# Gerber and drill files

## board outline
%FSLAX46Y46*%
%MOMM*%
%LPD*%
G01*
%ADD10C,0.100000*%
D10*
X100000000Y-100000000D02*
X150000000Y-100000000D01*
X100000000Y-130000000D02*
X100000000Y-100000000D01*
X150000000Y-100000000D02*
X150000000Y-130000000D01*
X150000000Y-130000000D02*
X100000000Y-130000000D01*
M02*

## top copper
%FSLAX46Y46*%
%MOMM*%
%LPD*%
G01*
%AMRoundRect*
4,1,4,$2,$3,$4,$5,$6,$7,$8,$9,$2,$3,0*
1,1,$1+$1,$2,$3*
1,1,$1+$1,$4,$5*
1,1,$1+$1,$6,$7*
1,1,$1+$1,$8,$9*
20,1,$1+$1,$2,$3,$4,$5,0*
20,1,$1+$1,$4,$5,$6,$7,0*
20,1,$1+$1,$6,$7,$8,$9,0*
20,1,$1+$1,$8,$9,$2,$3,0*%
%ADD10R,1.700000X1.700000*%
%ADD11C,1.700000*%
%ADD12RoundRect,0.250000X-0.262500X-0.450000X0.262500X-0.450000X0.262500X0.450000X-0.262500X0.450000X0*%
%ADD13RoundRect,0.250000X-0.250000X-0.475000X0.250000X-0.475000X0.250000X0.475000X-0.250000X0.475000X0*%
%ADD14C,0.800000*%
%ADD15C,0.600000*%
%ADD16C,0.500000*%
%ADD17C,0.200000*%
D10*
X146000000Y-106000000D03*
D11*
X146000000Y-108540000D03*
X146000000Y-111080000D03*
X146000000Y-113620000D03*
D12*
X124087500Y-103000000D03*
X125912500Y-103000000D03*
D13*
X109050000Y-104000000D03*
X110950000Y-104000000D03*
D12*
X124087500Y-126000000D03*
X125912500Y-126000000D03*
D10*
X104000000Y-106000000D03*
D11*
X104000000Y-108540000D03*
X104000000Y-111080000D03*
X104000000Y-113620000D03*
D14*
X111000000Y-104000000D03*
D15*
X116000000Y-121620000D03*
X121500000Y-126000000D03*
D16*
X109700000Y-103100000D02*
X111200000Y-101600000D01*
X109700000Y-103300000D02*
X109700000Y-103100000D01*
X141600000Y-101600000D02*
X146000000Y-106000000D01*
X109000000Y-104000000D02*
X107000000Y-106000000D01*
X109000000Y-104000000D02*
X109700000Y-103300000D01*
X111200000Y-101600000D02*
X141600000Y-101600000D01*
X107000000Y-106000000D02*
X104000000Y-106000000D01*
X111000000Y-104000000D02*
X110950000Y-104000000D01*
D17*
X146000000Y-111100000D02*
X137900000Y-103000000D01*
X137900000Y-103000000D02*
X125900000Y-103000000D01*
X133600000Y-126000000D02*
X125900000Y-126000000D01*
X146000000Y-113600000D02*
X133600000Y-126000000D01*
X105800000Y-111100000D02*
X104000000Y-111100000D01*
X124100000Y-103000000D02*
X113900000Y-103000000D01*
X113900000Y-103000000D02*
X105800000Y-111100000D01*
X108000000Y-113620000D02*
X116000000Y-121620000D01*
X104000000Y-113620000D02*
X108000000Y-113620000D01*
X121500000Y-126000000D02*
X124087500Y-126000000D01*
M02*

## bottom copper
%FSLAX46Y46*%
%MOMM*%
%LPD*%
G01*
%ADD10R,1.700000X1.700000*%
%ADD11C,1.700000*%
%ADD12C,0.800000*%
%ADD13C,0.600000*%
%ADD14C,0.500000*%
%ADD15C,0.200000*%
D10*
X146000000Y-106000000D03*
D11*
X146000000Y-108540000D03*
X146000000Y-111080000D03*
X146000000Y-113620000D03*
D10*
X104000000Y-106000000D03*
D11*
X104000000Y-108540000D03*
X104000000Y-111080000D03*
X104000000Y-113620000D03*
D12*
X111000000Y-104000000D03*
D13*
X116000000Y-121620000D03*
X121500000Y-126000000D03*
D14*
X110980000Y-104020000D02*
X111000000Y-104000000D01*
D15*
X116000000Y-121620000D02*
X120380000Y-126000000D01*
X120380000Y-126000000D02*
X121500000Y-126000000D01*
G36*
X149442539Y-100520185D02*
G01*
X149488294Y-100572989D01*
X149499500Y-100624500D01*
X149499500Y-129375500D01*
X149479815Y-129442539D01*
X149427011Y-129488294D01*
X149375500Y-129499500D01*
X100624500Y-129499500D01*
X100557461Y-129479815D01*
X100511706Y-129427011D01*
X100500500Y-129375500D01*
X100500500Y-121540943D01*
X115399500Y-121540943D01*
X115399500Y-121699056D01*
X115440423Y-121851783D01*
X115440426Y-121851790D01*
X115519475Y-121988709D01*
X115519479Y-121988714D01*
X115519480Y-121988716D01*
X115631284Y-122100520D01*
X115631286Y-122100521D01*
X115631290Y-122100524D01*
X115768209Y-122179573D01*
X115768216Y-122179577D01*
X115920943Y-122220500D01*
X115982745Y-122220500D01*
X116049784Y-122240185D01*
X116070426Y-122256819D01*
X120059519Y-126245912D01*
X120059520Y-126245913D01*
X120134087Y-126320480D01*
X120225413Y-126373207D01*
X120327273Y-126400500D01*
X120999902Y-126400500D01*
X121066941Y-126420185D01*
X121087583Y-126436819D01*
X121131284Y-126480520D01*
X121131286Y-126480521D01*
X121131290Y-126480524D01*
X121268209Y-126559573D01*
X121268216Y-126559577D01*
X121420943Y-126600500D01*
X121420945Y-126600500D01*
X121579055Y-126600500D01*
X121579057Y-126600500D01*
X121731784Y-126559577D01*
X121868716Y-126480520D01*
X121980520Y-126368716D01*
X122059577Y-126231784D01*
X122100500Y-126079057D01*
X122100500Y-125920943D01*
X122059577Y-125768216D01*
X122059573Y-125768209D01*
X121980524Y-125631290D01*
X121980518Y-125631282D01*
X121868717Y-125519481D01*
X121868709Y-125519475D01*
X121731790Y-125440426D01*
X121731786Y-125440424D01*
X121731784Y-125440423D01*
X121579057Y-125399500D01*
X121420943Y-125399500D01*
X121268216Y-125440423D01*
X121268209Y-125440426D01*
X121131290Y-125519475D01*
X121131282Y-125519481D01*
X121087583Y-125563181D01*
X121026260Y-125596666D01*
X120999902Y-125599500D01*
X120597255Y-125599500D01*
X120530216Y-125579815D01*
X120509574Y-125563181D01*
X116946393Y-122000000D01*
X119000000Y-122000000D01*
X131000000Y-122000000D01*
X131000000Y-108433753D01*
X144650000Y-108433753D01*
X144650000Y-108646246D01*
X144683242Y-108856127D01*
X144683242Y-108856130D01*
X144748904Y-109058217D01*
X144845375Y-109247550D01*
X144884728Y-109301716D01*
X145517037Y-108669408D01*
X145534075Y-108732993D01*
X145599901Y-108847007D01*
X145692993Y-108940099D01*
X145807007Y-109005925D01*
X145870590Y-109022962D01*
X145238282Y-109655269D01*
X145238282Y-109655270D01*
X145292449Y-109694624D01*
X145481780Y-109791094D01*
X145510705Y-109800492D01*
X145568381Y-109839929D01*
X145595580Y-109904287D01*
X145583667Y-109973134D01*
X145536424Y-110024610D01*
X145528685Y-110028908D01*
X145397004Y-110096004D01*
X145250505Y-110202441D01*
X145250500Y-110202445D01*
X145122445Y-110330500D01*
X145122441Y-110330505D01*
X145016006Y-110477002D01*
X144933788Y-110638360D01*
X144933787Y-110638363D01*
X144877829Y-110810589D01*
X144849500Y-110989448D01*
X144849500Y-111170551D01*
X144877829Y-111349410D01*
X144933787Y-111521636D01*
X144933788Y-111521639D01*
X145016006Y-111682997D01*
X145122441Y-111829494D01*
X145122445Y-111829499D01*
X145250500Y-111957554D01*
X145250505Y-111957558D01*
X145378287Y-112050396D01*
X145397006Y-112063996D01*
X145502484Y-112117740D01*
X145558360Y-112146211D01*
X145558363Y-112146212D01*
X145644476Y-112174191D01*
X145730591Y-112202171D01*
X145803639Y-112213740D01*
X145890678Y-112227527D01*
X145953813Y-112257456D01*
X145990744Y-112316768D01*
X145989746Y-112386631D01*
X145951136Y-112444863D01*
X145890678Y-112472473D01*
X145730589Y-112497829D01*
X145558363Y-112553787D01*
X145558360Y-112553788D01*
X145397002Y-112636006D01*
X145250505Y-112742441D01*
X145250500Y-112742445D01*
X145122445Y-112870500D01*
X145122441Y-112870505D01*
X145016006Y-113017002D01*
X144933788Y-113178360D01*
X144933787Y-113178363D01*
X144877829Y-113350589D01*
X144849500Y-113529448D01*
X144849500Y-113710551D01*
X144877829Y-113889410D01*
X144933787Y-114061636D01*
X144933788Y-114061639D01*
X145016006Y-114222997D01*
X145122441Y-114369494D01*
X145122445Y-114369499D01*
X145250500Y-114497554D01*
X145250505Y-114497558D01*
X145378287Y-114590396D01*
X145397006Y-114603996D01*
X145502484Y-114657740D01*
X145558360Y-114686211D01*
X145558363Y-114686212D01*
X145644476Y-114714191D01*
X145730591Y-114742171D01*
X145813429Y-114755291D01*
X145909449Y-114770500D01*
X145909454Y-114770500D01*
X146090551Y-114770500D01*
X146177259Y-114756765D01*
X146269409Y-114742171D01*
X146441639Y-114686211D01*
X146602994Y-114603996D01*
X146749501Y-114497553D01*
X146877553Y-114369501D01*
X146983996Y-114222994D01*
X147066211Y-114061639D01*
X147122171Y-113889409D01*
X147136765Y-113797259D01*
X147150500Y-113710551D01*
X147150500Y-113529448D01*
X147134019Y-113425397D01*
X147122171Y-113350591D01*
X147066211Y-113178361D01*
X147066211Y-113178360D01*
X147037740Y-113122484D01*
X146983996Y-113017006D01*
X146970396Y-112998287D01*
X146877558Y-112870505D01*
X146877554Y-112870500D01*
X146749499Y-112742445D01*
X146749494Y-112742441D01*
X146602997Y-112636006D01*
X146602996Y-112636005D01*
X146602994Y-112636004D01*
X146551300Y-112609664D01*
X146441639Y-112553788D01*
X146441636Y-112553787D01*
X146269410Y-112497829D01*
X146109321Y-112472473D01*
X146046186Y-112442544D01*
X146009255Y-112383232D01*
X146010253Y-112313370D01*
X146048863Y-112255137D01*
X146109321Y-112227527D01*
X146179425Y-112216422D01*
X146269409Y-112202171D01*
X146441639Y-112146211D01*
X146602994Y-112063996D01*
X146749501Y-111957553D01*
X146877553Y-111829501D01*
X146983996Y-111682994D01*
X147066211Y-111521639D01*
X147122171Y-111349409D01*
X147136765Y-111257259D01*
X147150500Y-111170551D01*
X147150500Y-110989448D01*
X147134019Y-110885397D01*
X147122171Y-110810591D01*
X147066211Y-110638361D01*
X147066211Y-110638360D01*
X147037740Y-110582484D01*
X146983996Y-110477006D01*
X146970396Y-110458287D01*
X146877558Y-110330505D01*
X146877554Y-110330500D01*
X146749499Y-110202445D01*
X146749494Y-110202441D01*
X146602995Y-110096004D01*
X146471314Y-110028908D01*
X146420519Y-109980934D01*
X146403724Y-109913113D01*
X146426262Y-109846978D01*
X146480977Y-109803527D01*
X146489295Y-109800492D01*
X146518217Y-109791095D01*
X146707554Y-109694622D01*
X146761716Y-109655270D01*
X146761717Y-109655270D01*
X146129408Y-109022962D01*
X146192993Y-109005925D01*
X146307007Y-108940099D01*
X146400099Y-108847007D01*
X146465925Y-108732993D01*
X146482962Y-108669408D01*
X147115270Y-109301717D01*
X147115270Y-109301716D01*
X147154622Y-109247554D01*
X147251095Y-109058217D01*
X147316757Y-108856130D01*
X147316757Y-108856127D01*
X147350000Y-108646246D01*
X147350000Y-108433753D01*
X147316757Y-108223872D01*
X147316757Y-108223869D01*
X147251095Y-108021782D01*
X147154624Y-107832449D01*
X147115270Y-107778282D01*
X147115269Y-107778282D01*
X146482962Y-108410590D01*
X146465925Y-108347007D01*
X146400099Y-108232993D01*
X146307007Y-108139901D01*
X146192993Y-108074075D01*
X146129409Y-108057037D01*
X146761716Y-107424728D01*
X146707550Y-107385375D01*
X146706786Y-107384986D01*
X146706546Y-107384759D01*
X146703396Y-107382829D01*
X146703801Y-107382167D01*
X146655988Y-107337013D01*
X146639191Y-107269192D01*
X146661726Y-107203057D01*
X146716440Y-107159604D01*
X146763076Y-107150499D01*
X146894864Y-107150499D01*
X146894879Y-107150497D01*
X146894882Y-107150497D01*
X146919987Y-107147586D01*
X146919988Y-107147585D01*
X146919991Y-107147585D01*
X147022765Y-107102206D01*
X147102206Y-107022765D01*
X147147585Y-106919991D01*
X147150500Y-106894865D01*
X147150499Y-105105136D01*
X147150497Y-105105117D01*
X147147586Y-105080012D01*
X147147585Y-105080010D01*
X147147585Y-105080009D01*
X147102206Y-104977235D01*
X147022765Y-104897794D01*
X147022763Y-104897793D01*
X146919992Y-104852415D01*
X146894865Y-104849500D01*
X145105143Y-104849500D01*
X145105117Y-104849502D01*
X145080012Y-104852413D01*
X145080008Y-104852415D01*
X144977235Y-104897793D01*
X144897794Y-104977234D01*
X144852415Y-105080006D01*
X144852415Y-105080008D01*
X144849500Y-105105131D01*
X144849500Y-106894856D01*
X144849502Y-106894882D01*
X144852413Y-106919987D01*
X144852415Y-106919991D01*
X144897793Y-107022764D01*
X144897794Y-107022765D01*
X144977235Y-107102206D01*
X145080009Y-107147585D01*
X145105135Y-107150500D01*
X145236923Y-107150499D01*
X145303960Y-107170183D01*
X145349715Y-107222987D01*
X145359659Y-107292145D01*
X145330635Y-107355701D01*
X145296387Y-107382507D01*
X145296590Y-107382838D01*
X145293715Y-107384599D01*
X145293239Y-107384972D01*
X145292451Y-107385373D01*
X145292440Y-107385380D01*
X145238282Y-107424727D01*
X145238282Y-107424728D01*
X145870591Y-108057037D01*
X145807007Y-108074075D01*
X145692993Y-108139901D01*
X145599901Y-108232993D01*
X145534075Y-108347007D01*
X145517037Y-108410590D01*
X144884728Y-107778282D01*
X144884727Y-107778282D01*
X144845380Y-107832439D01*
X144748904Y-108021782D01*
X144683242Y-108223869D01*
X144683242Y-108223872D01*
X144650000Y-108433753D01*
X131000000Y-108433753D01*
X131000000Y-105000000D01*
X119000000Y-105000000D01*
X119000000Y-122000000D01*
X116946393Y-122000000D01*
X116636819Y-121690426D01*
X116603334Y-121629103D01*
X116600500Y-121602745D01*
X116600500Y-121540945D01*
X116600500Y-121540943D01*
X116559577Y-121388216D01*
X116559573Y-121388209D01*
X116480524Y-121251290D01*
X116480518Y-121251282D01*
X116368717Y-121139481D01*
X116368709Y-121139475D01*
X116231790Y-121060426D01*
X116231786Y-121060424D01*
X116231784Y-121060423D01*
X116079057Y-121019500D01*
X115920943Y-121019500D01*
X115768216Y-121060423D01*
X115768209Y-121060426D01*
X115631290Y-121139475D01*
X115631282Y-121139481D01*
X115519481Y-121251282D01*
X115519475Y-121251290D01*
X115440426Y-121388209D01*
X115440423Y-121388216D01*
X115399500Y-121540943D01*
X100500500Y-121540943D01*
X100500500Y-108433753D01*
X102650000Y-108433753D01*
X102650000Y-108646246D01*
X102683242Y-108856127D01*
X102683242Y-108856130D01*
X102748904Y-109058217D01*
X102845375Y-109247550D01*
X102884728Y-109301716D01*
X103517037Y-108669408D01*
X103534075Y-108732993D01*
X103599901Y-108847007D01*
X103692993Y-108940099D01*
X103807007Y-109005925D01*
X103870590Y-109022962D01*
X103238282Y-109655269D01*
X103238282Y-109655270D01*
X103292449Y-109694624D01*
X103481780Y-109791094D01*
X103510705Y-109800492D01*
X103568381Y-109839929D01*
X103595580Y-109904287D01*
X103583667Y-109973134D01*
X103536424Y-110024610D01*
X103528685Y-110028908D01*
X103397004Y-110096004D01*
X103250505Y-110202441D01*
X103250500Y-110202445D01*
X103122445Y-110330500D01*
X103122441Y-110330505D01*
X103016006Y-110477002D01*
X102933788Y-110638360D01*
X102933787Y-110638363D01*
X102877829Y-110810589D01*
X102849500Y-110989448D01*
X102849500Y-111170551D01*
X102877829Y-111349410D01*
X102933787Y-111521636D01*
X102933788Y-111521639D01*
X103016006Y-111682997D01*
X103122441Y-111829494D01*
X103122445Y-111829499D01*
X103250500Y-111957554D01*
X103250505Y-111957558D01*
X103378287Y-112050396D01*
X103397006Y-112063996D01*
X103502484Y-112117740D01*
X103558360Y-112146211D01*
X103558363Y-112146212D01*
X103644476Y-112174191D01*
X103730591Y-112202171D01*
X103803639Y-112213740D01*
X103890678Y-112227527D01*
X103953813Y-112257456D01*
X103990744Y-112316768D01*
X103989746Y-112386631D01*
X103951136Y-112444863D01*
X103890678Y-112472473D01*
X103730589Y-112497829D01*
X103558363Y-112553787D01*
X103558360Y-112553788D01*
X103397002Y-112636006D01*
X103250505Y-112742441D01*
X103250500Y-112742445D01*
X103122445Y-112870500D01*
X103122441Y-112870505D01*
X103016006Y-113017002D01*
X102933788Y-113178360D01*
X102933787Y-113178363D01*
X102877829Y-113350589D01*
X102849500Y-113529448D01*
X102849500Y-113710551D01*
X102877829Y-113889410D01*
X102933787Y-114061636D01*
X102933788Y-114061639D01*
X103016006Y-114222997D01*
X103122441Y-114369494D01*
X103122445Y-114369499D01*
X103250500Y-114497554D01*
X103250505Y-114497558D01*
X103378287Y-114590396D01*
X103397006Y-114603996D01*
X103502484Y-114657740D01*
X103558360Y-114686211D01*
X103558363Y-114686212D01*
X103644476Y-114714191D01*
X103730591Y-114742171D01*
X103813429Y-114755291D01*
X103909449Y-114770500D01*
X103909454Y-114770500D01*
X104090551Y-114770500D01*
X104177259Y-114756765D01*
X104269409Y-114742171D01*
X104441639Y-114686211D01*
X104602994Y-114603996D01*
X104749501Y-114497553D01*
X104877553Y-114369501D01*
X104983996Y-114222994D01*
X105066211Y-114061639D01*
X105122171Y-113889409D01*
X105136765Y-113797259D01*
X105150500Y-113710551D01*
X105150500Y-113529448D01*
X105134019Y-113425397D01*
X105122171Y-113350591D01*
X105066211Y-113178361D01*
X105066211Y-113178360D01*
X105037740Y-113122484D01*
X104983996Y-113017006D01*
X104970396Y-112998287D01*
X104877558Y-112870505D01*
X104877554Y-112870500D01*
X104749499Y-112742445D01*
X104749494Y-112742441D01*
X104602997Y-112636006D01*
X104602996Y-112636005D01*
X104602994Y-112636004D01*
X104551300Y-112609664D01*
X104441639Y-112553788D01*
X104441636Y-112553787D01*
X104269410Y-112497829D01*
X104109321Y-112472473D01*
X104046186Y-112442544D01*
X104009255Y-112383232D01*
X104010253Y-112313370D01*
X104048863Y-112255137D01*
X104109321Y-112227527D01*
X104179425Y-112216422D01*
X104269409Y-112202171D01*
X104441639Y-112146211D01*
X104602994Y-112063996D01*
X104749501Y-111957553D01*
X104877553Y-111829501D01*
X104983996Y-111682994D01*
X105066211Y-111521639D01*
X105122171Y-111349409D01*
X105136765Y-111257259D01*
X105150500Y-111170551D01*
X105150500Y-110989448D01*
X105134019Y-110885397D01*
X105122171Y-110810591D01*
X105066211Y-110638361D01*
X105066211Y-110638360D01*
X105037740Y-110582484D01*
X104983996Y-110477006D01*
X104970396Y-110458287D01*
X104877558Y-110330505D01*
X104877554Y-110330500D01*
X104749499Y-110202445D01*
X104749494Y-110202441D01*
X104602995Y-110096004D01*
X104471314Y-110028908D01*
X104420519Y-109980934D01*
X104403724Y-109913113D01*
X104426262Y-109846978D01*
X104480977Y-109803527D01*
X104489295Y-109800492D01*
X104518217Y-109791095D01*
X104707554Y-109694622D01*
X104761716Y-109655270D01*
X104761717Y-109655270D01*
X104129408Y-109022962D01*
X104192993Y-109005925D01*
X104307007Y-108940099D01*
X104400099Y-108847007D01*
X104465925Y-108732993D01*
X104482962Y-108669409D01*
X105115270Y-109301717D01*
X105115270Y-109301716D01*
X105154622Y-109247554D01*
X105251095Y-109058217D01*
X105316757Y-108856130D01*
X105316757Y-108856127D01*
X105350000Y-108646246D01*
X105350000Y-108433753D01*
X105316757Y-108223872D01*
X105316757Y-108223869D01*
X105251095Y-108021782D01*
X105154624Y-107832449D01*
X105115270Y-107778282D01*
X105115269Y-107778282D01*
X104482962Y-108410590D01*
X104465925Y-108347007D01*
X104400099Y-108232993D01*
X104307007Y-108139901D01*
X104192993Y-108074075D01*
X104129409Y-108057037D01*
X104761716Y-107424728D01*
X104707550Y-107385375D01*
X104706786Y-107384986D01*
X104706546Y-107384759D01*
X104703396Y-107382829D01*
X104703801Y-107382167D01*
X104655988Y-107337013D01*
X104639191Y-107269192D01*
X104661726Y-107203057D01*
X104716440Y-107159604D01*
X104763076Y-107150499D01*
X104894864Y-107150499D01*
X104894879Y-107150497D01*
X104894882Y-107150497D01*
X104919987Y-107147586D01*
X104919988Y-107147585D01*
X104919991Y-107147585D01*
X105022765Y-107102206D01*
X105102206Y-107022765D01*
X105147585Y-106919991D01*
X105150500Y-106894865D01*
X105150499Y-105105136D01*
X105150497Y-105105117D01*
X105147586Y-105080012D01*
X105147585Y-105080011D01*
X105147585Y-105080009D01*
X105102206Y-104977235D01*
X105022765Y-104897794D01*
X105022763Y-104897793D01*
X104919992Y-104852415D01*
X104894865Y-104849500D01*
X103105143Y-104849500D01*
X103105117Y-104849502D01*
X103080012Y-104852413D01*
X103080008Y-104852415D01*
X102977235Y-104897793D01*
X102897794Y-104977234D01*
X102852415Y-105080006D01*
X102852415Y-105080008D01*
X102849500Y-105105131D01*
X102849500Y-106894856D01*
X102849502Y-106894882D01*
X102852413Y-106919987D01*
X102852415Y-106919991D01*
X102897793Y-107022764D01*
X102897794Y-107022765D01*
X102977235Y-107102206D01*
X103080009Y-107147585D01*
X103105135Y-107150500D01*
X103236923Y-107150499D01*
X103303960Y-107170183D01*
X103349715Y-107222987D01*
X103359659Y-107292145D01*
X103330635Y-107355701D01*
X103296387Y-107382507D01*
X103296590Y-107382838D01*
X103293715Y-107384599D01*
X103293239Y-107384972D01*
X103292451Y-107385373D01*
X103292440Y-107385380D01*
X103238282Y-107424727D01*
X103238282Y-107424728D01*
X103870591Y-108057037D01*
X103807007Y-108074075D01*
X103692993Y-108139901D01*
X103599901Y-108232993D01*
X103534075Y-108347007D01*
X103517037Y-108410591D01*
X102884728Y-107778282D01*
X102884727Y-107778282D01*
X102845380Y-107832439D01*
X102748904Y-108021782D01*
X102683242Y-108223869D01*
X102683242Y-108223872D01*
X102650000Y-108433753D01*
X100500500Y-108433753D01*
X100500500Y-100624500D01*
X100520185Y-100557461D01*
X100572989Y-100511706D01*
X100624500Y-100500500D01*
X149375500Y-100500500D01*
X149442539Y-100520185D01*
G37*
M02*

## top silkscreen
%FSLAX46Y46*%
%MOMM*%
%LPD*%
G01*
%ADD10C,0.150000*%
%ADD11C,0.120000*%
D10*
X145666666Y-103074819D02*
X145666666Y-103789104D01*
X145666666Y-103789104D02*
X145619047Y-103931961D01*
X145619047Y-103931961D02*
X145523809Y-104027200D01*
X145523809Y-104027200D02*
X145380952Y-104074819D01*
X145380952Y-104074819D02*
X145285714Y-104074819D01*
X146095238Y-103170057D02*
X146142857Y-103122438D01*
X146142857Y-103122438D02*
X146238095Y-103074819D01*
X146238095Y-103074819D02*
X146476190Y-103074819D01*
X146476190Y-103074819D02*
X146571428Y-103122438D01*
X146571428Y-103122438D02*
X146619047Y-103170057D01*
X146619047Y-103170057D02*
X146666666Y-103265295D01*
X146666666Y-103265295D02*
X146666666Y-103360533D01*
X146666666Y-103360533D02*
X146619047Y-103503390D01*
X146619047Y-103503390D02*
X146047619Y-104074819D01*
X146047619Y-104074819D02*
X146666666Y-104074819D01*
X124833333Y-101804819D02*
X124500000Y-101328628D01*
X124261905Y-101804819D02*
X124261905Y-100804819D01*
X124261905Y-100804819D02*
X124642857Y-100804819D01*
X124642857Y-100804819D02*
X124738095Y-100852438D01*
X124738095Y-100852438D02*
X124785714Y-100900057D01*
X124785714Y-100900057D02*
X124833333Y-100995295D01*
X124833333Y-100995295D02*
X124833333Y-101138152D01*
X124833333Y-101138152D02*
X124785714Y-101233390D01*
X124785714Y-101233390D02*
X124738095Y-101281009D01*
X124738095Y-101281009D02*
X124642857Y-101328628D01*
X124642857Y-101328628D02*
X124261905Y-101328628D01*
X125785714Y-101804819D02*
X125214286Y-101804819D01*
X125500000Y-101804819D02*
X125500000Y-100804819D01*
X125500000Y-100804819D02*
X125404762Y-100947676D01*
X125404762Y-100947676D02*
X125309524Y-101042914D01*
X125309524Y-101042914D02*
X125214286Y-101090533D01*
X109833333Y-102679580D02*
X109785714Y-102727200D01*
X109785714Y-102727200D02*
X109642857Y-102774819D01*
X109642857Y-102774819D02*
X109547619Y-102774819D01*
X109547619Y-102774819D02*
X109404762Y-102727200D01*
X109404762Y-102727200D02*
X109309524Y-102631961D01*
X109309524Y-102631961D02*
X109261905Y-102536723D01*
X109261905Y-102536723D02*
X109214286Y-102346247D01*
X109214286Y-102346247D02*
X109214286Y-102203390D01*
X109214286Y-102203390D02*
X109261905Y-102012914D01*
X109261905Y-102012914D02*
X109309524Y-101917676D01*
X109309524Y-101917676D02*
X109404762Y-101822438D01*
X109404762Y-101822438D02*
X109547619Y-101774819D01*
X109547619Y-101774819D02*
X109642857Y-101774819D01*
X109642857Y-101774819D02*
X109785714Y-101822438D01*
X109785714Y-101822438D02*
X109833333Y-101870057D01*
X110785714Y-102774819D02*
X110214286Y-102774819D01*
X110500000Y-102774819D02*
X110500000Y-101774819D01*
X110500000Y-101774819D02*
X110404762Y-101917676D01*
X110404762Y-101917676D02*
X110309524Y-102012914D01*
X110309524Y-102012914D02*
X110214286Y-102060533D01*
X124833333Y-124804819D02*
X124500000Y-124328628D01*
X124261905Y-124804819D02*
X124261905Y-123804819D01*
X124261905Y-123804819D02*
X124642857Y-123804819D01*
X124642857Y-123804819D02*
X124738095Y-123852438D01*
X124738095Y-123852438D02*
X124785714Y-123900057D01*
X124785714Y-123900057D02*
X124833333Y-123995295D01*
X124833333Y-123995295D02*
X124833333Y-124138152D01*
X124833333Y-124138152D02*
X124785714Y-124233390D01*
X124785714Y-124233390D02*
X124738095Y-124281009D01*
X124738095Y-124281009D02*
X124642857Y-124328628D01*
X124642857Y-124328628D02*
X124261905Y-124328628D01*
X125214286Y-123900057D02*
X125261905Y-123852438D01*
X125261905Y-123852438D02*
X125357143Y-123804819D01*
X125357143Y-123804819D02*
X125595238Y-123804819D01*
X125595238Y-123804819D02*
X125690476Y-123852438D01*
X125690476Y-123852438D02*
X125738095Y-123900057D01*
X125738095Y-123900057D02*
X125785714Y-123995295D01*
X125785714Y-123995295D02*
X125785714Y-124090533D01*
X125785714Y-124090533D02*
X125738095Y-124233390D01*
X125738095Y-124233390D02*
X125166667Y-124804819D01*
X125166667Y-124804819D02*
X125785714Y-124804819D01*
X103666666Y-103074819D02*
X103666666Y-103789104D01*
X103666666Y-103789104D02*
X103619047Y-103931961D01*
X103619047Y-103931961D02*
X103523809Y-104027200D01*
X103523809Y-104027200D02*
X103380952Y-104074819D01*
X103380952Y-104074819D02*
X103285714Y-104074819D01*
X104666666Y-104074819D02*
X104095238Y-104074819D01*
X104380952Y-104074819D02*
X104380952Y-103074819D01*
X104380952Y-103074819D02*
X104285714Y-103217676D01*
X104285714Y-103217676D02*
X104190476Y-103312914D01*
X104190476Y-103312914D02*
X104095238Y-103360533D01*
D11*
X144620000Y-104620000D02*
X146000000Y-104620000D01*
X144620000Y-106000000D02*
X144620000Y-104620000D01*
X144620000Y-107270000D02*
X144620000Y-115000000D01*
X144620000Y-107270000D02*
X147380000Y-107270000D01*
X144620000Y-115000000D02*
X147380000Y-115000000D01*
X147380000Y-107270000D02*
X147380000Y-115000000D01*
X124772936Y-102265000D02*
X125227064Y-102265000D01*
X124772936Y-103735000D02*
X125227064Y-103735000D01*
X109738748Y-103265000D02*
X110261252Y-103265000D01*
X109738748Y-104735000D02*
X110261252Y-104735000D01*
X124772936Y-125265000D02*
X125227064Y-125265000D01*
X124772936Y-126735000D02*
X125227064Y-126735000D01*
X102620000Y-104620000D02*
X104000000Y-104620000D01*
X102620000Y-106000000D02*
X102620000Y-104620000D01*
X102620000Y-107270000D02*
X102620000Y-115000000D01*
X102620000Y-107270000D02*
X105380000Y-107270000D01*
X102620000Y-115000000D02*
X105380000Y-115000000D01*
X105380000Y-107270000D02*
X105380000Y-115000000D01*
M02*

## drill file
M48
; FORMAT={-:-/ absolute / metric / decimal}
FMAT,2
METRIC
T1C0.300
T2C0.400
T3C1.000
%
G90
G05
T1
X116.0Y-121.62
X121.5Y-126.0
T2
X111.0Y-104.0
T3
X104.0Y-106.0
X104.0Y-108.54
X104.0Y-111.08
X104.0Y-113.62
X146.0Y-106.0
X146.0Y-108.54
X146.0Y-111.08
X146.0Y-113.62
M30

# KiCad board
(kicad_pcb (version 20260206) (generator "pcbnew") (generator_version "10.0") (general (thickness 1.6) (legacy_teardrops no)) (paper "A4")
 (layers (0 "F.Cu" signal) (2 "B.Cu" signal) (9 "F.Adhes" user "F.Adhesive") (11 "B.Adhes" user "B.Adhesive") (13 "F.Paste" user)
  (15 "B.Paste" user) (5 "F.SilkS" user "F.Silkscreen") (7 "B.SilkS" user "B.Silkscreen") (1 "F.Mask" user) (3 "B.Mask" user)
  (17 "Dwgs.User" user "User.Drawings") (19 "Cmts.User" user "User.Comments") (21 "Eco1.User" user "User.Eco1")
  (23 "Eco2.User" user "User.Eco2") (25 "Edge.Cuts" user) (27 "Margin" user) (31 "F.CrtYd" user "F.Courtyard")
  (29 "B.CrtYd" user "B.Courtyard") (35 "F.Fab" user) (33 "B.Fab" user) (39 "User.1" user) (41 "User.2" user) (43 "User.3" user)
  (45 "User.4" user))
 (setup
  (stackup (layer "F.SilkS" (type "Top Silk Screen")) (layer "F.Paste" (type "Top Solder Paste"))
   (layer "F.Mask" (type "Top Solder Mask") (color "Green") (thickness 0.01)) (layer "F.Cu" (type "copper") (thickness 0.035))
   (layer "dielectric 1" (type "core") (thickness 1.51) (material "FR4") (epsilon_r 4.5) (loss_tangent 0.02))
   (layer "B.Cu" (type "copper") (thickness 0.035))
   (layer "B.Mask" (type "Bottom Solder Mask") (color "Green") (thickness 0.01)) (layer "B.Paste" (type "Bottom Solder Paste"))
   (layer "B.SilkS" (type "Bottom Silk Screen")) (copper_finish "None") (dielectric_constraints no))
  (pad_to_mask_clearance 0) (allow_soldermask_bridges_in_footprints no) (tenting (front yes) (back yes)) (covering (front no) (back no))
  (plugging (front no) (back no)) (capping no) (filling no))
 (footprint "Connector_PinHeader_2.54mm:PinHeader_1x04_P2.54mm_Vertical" (layer "F.Cu") (at 146 106)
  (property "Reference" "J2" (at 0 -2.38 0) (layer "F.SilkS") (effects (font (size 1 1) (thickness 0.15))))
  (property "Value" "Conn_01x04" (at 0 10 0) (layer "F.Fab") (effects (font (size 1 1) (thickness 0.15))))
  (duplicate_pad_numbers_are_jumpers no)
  (fp_line (start -1.38 -1.38) (end 0 -1.38) (stroke (width 0.12) (type solid)) (layer "F.SilkS"))
  (fp_line (start -1.38 0) (end -1.38 -1.38) (stroke (width 0.12) (type solid)) (layer "F.SilkS"))
  (fp_line (start -1.38 1.27) (end -1.38 9) (stroke (width 0.12) (type solid)) (layer "F.SilkS"))
  (fp_line (start -1.38 1.27) (end 1.38 1.27) (stroke (width 0.12) (type solid)) (layer "F.SilkS"))
  (fp_line (start -1.38 9) (end 1.38 9) (stroke (width 0.12) (type solid)) (layer "F.SilkS"))
  (fp_line (start 1.38 1.27) (end 1.38 9) (stroke (width 0.12) (type solid)) (layer "F.SilkS"))
  (pad "1" thru_hole rect (at 0 0) (size 1.7 1.7) (drill 1) (layers "*.Cu" "*.Mask") (remove_unused_layers no) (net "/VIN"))
  (pad "2" thru_hole circle (at 0 2.54) (size 1.7 1.7) (drill 1) (layers "*.Cu" "*.Mask") (remove_unused_layers no) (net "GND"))
  (pad "3" thru_hole circle (at 0 5.08) (size 1.7 1.7) (drill 1) (layers "*.Cu" "*.Mask") (remove_unused_layers no) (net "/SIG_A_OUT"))
  (pad "4" thru_hole circle (at 0 7.62) (size 1.7 1.7) (drill 1) (layers "*.Cu" "*.Mask") (remove_unused_layers no) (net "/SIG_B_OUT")))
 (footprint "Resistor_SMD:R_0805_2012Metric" (layer "F.Cu") (at 125 103)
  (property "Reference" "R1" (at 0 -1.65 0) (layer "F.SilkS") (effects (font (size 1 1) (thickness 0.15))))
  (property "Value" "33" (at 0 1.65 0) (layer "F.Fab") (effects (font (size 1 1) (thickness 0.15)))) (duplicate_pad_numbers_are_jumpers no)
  (fp_line (start -0.227064 -0.735) (end 0.227064 -0.735) (stroke (width 0.12) (type solid)) (layer "F.SilkS"))
  (fp_line (start -0.227064 0.735) (end 0.227064 0.735) (stroke (width 0.12) (type solid)) (layer "F.SilkS"))
  (pad "1" smd roundrect (at -0.9125 0) (size 1.025 1.4) (layers "F.Cu" "F.Mask" "F.Paste") (roundrect_rratio 0.243902) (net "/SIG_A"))
  (pad "2" smd roundrect (at 0.9125 0) (size 1.025 1.4) (layers "F.Cu" "F.Mask" "F.Paste") (roundrect_rratio 0.243902) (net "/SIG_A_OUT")))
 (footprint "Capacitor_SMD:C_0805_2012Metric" (layer "F.Cu") (at 110 104)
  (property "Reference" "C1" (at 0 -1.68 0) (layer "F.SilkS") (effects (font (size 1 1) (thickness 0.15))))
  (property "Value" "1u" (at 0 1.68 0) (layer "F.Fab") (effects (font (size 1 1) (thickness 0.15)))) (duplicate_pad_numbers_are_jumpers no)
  (fp_line (start -0.261252 -0.735) (end 0.261252 -0.735) (stroke (width 0.12) (type solid)) (layer "F.SilkS"))
  (fp_line (start -0.261252 0.735) (end 0.261252 0.735) (stroke (width 0.12) (type solid)) (layer "F.SilkS"))
  (pad "1" smd roundrect (at -0.95 0) (size 1 1.45) (layers "F.Cu" "F.Mask" "F.Paste") (roundrect_rratio 0.25) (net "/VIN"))
  (pad "2" smd roundrect (at 0.95 0) (size 1 1.45) (layers "F.Cu" "F.Mask" "F.Paste") (roundrect_rratio 0.25) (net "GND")))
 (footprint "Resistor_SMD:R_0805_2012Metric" (layer "F.Cu") (at 125 126)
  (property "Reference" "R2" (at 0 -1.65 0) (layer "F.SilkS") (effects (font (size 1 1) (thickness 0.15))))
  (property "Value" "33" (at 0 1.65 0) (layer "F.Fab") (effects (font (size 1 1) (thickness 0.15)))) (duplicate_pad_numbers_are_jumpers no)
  (fp_line (start -0.227064 -0.735) (end 0.227064 -0.735) (stroke (width 0.12) (type solid)) (layer "F.SilkS"))
  (fp_line (start -0.227064 0.735) (end 0.227064 0.735) (stroke (width 0.12) (type solid)) (layer "F.SilkS"))
  (pad "1" smd roundrect (at -0.9125 0) (size 1.025 1.4) (layers "F.Cu" "F.Mask" "F.Paste") (roundrect_rratio 0.243902) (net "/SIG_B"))
  (pad "2" smd roundrect (at 0.9125 0) (size 1.025 1.4) (layers "F.Cu" "F.Mask" "F.Paste") (roundrect_rratio 0.243902) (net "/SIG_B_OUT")))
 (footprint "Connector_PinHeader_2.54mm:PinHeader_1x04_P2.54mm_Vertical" (layer "F.Cu") (at 104 106)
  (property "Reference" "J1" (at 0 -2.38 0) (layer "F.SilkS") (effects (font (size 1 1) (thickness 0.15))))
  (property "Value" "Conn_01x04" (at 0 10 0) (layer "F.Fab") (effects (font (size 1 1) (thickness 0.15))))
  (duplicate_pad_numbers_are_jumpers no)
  (fp_line (start -1.38 -1.38) (end 0 -1.38) (stroke (width 0.12) (type solid)) (layer "F.SilkS"))
  (fp_line (start -1.38 0) (end -1.38 -1.38) (stroke (width 0.12) (type solid)) (layer "F.SilkS"))
  (fp_line (start -1.38 1.27) (end -1.38 9) (stroke (width 0.12) (type solid)) (layer "F.SilkS"))
  (fp_line (start -1.38 1.27) (end 1.38 1.27) (stroke (width 0.12) (type solid)) (layer "F.SilkS"))
  (fp_line (start -1.38 9) (end 1.38 9) (stroke (width 0.12) (type solid)) (layer "F.SilkS"))
  (fp_line (start 1.38 1.27) (end 1.38 9) (stroke (width 0.12) (type solid)) (layer "F.SilkS"))
  (pad "1" thru_hole rect (at 0 0) (size 1.7 1.7) (drill 1) (layers "*.Cu" "*.Mask") (remove_unused_layers no) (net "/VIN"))
  (pad "2" thru_hole circle (at 0 2.54) (size 1.7 1.7) (drill 1) (layers "*.Cu" "*.Mask") (remove_unused_layers no) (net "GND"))
  (pad "3" thru_hole circle (at 0 5.08) (size 1.7 1.7) (drill 1) (layers "*.Cu" "*.Mask") (remove_unused_layers no) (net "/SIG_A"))
  (pad "4" thru_hole circle (at 0 7.62) (size 1.7 1.7) (drill 1) (layers "*.Cu" "*.Mask") (remove_unused_layers no) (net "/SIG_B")))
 (gr_line (start 100 100) (end 150 100) (stroke (width 0.1) (type default)) (layer "Edge.Cuts"))
 (gr_line (start 100 130) (end 100 100) (stroke (width 0.1) (type default)) (layer "Edge.Cuts"))
 (gr_line (start 150 100) (end 150 130) (stroke (width 0.1) (type default)) (layer "Edge.Cuts"))
 (gr_line (start 150 130) (end 100 130) (stroke (width 0.1) (type default)) (layer "Edge.Cuts"))
 (segment (start 109.7 103.1) (end 111.2 101.6) (width 0.5) (layer "F.Cu") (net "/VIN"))
 (segment (start 109.7 103.3) (end 109.7 103.1) (width 0.5) (layer "F.Cu") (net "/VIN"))
 (segment (start 141.6 101.6) (end 146 106) (width 0.5) (layer "F.Cu") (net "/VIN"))
 (segment (start 109 104) (end 107 106) (width 0.5) (layer "F.Cu") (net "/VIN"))
 (segment (start 109 104) (end 109.7 103.3) (width 0.5) (layer "F.Cu") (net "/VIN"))
 (segment (start 111.2 101.6) (end 141.6 101.6) (width 0.5) (layer "F.Cu") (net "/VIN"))
 (segment (start 107 106) (end 104 106) (width 0.5) (layer "F.Cu") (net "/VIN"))
 (segment (start 111 104) (end 110.95 104) (width 0.5) (layer "F.Cu") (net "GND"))
 (via (at 111 104) (size 0.8) (drill 0.4) (layers "F.Cu" "B.Cu") (capping yes) (filling yes) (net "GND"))
 (segment (start 110.98 104.02) (end 111 104) (width 0.5) (layer "B.Cu") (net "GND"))
 (segment (start 146 111.1) (end 137.9 103) (width 0.2) (layer "F.Cu") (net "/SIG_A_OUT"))
 (segment (start 137.9 103) (end 125.9 103) (width 0.2) (layer "F.Cu") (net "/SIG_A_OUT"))
 (segment (start 133.6 126) (end 125.9 126) (width 0.2) (layer "F.Cu") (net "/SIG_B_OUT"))
 (segment (start 146 113.6) (end 133.6 126) (width 0.2) (layer "F.Cu") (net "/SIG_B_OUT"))
 (segment (start 105.8 111.1) (end 104 111.1) (width 0.2) (layer "F.Cu") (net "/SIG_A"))
 (segment (start 124.1 103) (end 113.9 103) (width 0.2) (layer "F.Cu") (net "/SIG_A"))
 (segment (start 113.9 103) (end 105.8 111.1) (width 0.2) (layer "F.Cu") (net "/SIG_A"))
 (segment (start 108 113.62) (end 116 121.62) (width 0.2) (locked yes) (layer "F.Cu") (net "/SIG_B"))
 (segment (start 104 113.62) (end 108 113.62) (width 0.2) (locked yes) (layer "F.Cu") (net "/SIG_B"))
 (segment (start 121.5 126) (end 124.0875 126) (width 0.2) (locked yes) (layer "F.Cu") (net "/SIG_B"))
 (via (at 116 121.62) (size 0.6) (drill 0.3) (layers "F.Cu" "B.Cu") (locked yes) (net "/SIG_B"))
 (via (at 121.5 126) (size 0.6) (drill 0.3) (layers "F.Cu" "B.Cu") (locked yes) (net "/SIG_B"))
 (segment (start 116 121.62) (end 120.38 126) (width 0.2) (locked yes) (layer "B.Cu") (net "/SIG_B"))
 (segment (start 120.38 126) (end 121.5 126) (width 0.2) (locked yes) (layer "B.Cu") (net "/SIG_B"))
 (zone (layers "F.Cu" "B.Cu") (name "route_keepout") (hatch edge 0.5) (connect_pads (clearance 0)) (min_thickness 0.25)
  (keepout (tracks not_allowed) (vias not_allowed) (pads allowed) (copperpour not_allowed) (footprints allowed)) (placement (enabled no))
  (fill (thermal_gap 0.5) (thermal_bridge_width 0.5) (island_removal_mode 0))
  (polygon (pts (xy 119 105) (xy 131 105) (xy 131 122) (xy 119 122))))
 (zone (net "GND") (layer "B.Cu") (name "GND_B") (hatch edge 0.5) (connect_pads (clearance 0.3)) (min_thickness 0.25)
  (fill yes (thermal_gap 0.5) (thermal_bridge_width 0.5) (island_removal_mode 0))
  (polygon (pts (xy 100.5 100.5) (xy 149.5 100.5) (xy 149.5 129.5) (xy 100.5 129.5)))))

